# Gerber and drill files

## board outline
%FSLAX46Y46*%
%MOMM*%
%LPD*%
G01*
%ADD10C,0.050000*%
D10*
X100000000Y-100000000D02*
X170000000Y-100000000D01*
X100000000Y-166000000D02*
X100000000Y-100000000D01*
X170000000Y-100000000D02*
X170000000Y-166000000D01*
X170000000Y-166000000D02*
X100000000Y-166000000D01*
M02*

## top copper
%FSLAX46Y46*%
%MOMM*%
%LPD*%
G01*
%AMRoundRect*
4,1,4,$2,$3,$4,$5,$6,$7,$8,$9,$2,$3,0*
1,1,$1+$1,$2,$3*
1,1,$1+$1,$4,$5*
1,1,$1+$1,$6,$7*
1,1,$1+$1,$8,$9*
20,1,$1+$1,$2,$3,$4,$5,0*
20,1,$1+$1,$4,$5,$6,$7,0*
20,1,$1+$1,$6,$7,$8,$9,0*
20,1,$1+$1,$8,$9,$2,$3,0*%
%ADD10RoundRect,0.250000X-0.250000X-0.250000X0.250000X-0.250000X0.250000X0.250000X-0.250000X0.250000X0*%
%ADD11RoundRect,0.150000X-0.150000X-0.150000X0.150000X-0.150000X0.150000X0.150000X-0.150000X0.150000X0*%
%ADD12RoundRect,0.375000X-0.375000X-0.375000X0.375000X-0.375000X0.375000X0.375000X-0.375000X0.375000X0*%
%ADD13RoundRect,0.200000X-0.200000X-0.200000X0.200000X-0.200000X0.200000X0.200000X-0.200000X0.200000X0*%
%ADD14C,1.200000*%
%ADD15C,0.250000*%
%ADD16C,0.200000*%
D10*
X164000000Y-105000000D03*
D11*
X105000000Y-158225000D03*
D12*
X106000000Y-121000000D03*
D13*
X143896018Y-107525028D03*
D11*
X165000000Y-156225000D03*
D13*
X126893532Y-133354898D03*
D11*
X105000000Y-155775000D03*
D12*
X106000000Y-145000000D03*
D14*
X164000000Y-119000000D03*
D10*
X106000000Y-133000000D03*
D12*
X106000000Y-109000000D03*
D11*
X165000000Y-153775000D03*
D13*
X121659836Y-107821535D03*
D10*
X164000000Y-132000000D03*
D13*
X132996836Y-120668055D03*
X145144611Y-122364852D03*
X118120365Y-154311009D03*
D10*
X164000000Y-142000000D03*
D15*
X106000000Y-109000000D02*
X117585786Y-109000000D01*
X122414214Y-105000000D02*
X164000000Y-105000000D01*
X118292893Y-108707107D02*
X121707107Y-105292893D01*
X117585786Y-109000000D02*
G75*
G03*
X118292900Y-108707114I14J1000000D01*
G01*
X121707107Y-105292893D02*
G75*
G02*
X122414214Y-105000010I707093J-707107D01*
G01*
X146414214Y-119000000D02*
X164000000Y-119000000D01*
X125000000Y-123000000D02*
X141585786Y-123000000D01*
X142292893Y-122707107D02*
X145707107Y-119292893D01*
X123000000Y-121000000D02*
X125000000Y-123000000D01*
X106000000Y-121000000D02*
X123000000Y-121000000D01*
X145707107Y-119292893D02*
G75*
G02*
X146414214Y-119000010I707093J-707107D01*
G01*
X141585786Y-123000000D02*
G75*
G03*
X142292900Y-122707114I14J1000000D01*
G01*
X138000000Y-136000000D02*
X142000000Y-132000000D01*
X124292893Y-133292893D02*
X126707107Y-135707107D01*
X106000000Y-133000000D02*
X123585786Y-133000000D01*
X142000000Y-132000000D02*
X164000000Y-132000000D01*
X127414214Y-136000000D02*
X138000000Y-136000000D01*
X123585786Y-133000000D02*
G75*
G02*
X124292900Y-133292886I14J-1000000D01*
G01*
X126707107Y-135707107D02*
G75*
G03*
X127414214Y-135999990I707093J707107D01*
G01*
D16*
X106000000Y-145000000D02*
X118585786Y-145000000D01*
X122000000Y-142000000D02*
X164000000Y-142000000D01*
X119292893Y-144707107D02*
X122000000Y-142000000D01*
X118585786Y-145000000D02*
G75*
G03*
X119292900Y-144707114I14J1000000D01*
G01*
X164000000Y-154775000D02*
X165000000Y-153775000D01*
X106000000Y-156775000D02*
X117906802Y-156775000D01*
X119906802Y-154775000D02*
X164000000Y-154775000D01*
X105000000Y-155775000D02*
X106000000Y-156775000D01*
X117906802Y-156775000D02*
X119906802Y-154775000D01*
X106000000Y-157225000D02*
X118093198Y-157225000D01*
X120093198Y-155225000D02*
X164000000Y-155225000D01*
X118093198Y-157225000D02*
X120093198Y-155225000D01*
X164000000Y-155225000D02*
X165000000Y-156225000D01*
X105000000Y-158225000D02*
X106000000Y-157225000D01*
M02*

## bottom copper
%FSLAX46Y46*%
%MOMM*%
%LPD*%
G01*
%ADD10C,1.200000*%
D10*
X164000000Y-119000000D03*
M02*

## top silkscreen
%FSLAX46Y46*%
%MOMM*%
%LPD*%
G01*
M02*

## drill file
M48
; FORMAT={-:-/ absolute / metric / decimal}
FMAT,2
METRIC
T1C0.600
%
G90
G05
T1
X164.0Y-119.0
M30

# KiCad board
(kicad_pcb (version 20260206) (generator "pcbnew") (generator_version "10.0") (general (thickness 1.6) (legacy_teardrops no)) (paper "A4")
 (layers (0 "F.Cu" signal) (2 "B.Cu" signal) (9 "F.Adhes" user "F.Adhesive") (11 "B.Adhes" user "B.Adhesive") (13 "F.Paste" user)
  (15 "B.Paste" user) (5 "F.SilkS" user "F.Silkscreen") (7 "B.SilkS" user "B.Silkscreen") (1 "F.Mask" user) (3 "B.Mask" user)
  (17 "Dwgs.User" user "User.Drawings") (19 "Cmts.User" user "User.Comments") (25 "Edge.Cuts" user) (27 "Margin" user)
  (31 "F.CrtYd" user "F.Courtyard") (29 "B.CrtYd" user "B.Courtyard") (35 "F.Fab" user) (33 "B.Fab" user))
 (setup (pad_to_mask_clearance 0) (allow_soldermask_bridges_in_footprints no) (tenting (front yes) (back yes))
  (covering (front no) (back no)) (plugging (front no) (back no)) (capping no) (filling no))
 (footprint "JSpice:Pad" (layer "F.Cu") (at 164 105)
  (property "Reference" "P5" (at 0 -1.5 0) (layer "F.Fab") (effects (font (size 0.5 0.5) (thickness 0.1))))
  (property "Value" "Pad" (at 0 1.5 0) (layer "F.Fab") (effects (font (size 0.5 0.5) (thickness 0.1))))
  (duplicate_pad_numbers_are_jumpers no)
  (pad "1" smd roundrect (at 0 0) (size 1 1) (layers "F.Cu" "F.Mask") (roundrect_rratio 0.25) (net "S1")))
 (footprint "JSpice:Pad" (layer "F.Cu") (at 105 158.225)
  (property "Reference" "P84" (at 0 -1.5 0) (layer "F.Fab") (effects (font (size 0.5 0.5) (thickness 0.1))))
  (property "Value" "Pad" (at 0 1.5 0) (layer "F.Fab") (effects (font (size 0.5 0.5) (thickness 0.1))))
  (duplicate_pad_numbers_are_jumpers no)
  (pad "1" smd roundrect (at 0 0) (size 0.6 0.6) (layers "F.Cu" "F.Mask") (roundrect_rratio 0.25) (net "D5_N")))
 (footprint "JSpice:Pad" (layer "F.Cu") (at 106 121)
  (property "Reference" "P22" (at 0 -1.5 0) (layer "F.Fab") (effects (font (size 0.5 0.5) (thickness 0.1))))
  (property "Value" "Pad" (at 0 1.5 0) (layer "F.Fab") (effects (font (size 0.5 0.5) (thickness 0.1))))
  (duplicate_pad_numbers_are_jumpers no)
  (pad "1" smd roundrect (at 0 0) (size 1.5 1.5) (layers "F.Cu" "F.Mask") (roundrect_rratio 0.25) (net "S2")))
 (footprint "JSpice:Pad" (layer "F.Cu") (at 143.896018 107.525028)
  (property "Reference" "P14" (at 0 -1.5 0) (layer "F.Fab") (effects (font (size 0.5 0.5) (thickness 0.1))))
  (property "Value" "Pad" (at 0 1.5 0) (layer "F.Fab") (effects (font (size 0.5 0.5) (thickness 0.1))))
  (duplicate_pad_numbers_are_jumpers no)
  (pad "1" smd roundrect (at 0 0) (size 0.8 0.8) (layers "F.Cu" "F.Mask") (roundrect_rratio 0.25) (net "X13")))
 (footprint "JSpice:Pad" (layer "F.Cu") (at 165 156.225)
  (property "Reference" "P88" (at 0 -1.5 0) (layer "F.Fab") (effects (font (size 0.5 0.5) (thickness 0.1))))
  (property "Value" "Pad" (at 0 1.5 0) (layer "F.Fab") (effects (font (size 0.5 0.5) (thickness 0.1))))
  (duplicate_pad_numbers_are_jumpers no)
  (pad "1" smd roundrect (at 0 0) (size 0.6 0.6) (layers "F.Cu" "F.Mask") (roundrect_rratio 0.25) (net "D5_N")))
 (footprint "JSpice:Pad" (layer "F.Cu") (at 126.893532 133.354898)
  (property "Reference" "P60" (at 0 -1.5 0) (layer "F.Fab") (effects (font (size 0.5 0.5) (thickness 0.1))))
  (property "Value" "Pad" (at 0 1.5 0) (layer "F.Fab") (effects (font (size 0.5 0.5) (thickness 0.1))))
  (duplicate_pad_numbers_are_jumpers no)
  (pad "1" smd roundrect (at 0 0) (size 0.8 0.8) (layers "F.Cu" "F.Mask") (roundrect_rratio 0.25) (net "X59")))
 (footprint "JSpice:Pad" (layer "F.Cu") (at 105 155.775)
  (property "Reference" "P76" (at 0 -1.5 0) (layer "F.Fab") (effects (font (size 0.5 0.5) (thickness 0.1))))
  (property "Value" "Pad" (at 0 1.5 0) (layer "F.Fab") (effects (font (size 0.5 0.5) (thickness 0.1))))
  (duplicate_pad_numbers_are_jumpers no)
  (pad "1" smd roundrect (at 0 0) (size 0.6 0.6) (layers "F.Cu" "F.Mask") (roundrect_rratio 0.25) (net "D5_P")))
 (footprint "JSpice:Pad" (layer "F.Cu") (at 106 145)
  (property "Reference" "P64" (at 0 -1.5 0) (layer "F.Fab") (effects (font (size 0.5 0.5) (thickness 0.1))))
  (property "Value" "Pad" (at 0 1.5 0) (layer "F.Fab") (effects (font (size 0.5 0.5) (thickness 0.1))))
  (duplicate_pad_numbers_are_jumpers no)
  (pad "1" smd roundrect (at 0 0) (size 1.5 1.5) (layers "F.Cu" "F.Mask") (roundrect_rratio 0.25) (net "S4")))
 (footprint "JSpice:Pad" (layer "F.Cu") (at 164 119)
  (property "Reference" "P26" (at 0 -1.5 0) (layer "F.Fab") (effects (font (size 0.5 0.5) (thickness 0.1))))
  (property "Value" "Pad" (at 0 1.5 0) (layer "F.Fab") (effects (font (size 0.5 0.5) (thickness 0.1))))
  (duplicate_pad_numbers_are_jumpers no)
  (pad "1" thru_hole circle (at 0 0) (size 1.2 1.2) (drill 0.6) (layers "*.Cu" "*.Mask") (remove_unused_layers no) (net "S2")))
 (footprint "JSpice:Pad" (layer "F.Cu") (at 106 133)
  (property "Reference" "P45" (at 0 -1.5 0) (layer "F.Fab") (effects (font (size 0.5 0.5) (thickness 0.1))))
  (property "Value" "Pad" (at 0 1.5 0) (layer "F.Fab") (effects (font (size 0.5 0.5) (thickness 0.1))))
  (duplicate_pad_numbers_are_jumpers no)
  (pad "1" smd roundrect (at 0 0) (size 1 1) (layers "F.Cu" "F.Mask") (roundrect_rratio 0.25) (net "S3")))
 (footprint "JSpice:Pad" (layer "F.Cu") (at 106 109)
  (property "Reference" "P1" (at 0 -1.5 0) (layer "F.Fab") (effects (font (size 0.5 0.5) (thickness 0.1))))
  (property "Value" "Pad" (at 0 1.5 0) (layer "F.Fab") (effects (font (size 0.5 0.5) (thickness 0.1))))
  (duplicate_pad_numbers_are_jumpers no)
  (pad "1" smd roundrect (at 0 0) (size 1.5 1.5) (layers "F.Cu" "F.Mask") (roundrect_rratio 0.25) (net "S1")))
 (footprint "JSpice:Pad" (layer "F.Cu") (at 165 153.775)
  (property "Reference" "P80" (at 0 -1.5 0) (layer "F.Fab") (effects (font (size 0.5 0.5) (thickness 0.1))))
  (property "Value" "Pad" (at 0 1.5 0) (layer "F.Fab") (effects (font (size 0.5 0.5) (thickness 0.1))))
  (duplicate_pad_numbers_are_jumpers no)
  (pad "1" smd roundrect (at 0 0) (size 0.6 0.6) (layers "F.Cu" "F.Mask") (roundrect_rratio 0.25) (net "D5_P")))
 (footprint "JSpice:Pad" (layer "F.Cu") (at 121.659836 107.821535)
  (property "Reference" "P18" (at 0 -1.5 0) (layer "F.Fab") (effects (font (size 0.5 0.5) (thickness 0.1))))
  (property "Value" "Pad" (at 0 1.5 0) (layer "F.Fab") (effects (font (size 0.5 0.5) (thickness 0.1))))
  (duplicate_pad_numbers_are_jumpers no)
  (pad "1" smd roundrect (at 0 0) (size 0.8 0.8) (layers "F.Cu" "F.Mask") (roundrect_rratio 0.25) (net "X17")))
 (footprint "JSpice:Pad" (layer "F.Cu") (at 164 132)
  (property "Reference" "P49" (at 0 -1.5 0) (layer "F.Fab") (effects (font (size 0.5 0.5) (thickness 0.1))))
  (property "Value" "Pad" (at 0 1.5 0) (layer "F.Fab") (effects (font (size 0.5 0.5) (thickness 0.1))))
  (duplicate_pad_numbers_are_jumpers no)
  (pad "1" smd roundrect (at 0 0) (size 1 1) (layers "F.Cu" "F.Mask") (roundrect_rratio 0.25) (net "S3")))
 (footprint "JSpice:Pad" (layer "F.Cu") (at 132.996836 120.668055)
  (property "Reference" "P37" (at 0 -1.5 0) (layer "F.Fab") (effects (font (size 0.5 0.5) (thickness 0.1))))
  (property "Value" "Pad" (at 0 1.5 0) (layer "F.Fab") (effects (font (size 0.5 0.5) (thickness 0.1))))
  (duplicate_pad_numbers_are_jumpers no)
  (pad "1" smd roundrect (at 0 0) (size 0.8 0.8) (layers "F.Cu" "F.Mask") (roundrect_rratio 0.25) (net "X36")))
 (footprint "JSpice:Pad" (layer "F.Cu") (at 145.144611 122.364852)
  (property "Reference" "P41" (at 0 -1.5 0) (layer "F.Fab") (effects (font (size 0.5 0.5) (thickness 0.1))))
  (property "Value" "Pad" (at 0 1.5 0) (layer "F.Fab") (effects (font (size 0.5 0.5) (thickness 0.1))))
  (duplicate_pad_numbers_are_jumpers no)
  (pad "1" smd roundrect (at 0 0) (size 0.8 0.8) (layers "F.Cu" "F.Mask") (roundrect_rratio 0.25) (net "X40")))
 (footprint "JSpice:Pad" (layer "F.Cu") (at 118.120365 154.311009)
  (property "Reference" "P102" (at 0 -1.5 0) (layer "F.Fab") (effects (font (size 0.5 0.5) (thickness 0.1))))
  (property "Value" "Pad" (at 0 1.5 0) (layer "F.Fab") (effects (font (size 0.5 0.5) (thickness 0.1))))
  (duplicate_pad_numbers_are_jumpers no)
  (pad "1" smd roundrect (at 0 0) (size 0.8 0.8) (layers "F.Cu" "F.Mask") (roundrect_rratio 0.25) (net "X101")))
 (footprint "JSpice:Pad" (layer "F.Cu") (at 164 142)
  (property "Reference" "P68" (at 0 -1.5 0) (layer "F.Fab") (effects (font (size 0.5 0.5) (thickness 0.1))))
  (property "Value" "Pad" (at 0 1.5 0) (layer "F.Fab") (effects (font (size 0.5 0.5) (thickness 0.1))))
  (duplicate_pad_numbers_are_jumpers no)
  (pad "1" smd roundrect (at 0 0) (size 1 1) (layers "F.Cu" "F.Mask") (roundrect_rratio 0.25) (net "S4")))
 (gr_line (start 100 100) (end 170 100) (stroke (width 0.05) (type default)) (layer "Edge.Cuts"))
 (gr_line (start 100 166) (end 100 100) (stroke (width 0.05) (type default)) (layer "Edge.Cuts"))
 (gr_line (start 170 100) (end 170 166) (stroke (width 0.05) (type default)) (layer "Edge.Cuts"))
 (gr_line (start 170 166) (end 100 166) (stroke (width 0.05) (type default)) (layer "Edge.Cuts"))
 (segment (start 106 109) (end 117.585786 109) (width 0.25) (layer "F.Cu") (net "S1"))
 (segment (start 122.414214 105) (end 164 105) (width 0.25) (layer "F.Cu") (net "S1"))
 (segment (start 118.292893 108.707107) (end 121.707107 105.292893) (width 0.25) (layer "F.Cu") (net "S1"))
 (arc (start 117.585786 109) (mid 117.96847 108.92388) (end 118.292893 108.707107) (width 0.25) (layer "F.Cu") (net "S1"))
 (arc (start 121.707107 105.292893) (mid 122.03153 105.07612) (end 122.414214 105) (width 0.25) (layer "F.Cu") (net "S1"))
 (segment (start 146.414214 119) (end 164 119) (width 0.25) (layer "F.Cu") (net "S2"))
 (segment (start 125 123) (end 141.585786 123) (width 0.25) (layer "F.Cu") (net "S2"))
 (segment (start 142.292893 122.707107) (end 145.707107 119.292893) (width 0.25) (layer "F.Cu") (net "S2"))
 (segment (start 123 121) (end 125 123) (width 0.25) (layer "F.Cu") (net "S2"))
 (segment (start 106 121) (end 123 121) (width 0.25) (layer "F.Cu") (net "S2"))
 (arc (start 145.707107 119.292893) (mid 146.03153 119.07612) (end 146.414214 119) (width 0.25) (layer "F.Cu") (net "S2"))
 (arc (start 141.585786 123) (mid 141.96847 122.92388) (end 142.292893 122.707107) (width 0.25) (layer "F.Cu") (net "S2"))
 (segment (start 138 136) (end 142 132) (width 0.25) (layer "F.Cu") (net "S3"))
 (segment (start 124.292893 133.292893) (end 126.707107 135.707107) (width 0.25) (layer "F.Cu") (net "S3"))
 (segment (start 106 133) (end 123.585786 133) (width 0.25) (layer "F.Cu") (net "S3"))
 (segment (start 142 132) (end 164 132) (width 0.25) (layer "F.Cu") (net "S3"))
 (segment (start 127.414214 136) (end 138 136) (width 0.25) (layer "F.Cu") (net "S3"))
 (arc (start 123.585786 133) (mid 123.96847 133.07612) (end 124.292893 133.292893) (width 0.25) (layer "F.Cu") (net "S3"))
 (arc (start 126.707107 135.707107) (mid 127.03153 135.92388) (end 127.414214 136) (width 0.25) (layer "F.Cu") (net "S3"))
 (segment (start 106 145) (end 118.585786 145) (width 0.2) (layer "F.Cu") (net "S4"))
 (segment (start 122 142) (end 164 142) (width 0.2) (layer "F.Cu") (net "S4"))
 (segment (start 119.292893 144.707107) (end 122 142) (width 0.2) (layer "F.Cu") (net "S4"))
 (arc (start 118.585786 145) (mid 118.96847 144.92388) (end 119.292893 144.707107) (width 0.2) (layer "F.Cu") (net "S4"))
 (segment (start 164 154.775) (end 165 153.775) (width 0.2) (layer "F.Cu") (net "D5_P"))
 (segment (start 106 156.775) (end 117.906802 156.775) (width 0.2) (layer "F.Cu") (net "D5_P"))
 (segment (start 119.906802 154.775) (end 164 154.775) (width 0.2) (layer "F.Cu") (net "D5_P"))
 (segment (start 105 155.775) (end 106 156.775) (width 0.2) (layer "F.Cu") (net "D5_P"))
 (segment (start 117.906802 156.775) (end 119.906802 154.775) (width 0.2) (layer "F.Cu") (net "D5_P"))
 (segment (start 106 157.225) (end 118.093198 157.225) (width 0.2) (layer "F.Cu") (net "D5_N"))
 (segment (start 120.093198 155.225) (end 164 155.225) (width 0.2) (layer "F.Cu") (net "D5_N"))
 (segment (start 118.093198 157.225) (end 120.093198 155.225) (width 0.2) (layer "F.Cu") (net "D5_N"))
 (segment (start 164 155.225) (end 165 156.225) (width 0.2) (layer "F.Cu") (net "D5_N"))
 (segment (start 105 158.225) (end 106 157.225) (width 0.2) (layer "F.Cu") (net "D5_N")))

